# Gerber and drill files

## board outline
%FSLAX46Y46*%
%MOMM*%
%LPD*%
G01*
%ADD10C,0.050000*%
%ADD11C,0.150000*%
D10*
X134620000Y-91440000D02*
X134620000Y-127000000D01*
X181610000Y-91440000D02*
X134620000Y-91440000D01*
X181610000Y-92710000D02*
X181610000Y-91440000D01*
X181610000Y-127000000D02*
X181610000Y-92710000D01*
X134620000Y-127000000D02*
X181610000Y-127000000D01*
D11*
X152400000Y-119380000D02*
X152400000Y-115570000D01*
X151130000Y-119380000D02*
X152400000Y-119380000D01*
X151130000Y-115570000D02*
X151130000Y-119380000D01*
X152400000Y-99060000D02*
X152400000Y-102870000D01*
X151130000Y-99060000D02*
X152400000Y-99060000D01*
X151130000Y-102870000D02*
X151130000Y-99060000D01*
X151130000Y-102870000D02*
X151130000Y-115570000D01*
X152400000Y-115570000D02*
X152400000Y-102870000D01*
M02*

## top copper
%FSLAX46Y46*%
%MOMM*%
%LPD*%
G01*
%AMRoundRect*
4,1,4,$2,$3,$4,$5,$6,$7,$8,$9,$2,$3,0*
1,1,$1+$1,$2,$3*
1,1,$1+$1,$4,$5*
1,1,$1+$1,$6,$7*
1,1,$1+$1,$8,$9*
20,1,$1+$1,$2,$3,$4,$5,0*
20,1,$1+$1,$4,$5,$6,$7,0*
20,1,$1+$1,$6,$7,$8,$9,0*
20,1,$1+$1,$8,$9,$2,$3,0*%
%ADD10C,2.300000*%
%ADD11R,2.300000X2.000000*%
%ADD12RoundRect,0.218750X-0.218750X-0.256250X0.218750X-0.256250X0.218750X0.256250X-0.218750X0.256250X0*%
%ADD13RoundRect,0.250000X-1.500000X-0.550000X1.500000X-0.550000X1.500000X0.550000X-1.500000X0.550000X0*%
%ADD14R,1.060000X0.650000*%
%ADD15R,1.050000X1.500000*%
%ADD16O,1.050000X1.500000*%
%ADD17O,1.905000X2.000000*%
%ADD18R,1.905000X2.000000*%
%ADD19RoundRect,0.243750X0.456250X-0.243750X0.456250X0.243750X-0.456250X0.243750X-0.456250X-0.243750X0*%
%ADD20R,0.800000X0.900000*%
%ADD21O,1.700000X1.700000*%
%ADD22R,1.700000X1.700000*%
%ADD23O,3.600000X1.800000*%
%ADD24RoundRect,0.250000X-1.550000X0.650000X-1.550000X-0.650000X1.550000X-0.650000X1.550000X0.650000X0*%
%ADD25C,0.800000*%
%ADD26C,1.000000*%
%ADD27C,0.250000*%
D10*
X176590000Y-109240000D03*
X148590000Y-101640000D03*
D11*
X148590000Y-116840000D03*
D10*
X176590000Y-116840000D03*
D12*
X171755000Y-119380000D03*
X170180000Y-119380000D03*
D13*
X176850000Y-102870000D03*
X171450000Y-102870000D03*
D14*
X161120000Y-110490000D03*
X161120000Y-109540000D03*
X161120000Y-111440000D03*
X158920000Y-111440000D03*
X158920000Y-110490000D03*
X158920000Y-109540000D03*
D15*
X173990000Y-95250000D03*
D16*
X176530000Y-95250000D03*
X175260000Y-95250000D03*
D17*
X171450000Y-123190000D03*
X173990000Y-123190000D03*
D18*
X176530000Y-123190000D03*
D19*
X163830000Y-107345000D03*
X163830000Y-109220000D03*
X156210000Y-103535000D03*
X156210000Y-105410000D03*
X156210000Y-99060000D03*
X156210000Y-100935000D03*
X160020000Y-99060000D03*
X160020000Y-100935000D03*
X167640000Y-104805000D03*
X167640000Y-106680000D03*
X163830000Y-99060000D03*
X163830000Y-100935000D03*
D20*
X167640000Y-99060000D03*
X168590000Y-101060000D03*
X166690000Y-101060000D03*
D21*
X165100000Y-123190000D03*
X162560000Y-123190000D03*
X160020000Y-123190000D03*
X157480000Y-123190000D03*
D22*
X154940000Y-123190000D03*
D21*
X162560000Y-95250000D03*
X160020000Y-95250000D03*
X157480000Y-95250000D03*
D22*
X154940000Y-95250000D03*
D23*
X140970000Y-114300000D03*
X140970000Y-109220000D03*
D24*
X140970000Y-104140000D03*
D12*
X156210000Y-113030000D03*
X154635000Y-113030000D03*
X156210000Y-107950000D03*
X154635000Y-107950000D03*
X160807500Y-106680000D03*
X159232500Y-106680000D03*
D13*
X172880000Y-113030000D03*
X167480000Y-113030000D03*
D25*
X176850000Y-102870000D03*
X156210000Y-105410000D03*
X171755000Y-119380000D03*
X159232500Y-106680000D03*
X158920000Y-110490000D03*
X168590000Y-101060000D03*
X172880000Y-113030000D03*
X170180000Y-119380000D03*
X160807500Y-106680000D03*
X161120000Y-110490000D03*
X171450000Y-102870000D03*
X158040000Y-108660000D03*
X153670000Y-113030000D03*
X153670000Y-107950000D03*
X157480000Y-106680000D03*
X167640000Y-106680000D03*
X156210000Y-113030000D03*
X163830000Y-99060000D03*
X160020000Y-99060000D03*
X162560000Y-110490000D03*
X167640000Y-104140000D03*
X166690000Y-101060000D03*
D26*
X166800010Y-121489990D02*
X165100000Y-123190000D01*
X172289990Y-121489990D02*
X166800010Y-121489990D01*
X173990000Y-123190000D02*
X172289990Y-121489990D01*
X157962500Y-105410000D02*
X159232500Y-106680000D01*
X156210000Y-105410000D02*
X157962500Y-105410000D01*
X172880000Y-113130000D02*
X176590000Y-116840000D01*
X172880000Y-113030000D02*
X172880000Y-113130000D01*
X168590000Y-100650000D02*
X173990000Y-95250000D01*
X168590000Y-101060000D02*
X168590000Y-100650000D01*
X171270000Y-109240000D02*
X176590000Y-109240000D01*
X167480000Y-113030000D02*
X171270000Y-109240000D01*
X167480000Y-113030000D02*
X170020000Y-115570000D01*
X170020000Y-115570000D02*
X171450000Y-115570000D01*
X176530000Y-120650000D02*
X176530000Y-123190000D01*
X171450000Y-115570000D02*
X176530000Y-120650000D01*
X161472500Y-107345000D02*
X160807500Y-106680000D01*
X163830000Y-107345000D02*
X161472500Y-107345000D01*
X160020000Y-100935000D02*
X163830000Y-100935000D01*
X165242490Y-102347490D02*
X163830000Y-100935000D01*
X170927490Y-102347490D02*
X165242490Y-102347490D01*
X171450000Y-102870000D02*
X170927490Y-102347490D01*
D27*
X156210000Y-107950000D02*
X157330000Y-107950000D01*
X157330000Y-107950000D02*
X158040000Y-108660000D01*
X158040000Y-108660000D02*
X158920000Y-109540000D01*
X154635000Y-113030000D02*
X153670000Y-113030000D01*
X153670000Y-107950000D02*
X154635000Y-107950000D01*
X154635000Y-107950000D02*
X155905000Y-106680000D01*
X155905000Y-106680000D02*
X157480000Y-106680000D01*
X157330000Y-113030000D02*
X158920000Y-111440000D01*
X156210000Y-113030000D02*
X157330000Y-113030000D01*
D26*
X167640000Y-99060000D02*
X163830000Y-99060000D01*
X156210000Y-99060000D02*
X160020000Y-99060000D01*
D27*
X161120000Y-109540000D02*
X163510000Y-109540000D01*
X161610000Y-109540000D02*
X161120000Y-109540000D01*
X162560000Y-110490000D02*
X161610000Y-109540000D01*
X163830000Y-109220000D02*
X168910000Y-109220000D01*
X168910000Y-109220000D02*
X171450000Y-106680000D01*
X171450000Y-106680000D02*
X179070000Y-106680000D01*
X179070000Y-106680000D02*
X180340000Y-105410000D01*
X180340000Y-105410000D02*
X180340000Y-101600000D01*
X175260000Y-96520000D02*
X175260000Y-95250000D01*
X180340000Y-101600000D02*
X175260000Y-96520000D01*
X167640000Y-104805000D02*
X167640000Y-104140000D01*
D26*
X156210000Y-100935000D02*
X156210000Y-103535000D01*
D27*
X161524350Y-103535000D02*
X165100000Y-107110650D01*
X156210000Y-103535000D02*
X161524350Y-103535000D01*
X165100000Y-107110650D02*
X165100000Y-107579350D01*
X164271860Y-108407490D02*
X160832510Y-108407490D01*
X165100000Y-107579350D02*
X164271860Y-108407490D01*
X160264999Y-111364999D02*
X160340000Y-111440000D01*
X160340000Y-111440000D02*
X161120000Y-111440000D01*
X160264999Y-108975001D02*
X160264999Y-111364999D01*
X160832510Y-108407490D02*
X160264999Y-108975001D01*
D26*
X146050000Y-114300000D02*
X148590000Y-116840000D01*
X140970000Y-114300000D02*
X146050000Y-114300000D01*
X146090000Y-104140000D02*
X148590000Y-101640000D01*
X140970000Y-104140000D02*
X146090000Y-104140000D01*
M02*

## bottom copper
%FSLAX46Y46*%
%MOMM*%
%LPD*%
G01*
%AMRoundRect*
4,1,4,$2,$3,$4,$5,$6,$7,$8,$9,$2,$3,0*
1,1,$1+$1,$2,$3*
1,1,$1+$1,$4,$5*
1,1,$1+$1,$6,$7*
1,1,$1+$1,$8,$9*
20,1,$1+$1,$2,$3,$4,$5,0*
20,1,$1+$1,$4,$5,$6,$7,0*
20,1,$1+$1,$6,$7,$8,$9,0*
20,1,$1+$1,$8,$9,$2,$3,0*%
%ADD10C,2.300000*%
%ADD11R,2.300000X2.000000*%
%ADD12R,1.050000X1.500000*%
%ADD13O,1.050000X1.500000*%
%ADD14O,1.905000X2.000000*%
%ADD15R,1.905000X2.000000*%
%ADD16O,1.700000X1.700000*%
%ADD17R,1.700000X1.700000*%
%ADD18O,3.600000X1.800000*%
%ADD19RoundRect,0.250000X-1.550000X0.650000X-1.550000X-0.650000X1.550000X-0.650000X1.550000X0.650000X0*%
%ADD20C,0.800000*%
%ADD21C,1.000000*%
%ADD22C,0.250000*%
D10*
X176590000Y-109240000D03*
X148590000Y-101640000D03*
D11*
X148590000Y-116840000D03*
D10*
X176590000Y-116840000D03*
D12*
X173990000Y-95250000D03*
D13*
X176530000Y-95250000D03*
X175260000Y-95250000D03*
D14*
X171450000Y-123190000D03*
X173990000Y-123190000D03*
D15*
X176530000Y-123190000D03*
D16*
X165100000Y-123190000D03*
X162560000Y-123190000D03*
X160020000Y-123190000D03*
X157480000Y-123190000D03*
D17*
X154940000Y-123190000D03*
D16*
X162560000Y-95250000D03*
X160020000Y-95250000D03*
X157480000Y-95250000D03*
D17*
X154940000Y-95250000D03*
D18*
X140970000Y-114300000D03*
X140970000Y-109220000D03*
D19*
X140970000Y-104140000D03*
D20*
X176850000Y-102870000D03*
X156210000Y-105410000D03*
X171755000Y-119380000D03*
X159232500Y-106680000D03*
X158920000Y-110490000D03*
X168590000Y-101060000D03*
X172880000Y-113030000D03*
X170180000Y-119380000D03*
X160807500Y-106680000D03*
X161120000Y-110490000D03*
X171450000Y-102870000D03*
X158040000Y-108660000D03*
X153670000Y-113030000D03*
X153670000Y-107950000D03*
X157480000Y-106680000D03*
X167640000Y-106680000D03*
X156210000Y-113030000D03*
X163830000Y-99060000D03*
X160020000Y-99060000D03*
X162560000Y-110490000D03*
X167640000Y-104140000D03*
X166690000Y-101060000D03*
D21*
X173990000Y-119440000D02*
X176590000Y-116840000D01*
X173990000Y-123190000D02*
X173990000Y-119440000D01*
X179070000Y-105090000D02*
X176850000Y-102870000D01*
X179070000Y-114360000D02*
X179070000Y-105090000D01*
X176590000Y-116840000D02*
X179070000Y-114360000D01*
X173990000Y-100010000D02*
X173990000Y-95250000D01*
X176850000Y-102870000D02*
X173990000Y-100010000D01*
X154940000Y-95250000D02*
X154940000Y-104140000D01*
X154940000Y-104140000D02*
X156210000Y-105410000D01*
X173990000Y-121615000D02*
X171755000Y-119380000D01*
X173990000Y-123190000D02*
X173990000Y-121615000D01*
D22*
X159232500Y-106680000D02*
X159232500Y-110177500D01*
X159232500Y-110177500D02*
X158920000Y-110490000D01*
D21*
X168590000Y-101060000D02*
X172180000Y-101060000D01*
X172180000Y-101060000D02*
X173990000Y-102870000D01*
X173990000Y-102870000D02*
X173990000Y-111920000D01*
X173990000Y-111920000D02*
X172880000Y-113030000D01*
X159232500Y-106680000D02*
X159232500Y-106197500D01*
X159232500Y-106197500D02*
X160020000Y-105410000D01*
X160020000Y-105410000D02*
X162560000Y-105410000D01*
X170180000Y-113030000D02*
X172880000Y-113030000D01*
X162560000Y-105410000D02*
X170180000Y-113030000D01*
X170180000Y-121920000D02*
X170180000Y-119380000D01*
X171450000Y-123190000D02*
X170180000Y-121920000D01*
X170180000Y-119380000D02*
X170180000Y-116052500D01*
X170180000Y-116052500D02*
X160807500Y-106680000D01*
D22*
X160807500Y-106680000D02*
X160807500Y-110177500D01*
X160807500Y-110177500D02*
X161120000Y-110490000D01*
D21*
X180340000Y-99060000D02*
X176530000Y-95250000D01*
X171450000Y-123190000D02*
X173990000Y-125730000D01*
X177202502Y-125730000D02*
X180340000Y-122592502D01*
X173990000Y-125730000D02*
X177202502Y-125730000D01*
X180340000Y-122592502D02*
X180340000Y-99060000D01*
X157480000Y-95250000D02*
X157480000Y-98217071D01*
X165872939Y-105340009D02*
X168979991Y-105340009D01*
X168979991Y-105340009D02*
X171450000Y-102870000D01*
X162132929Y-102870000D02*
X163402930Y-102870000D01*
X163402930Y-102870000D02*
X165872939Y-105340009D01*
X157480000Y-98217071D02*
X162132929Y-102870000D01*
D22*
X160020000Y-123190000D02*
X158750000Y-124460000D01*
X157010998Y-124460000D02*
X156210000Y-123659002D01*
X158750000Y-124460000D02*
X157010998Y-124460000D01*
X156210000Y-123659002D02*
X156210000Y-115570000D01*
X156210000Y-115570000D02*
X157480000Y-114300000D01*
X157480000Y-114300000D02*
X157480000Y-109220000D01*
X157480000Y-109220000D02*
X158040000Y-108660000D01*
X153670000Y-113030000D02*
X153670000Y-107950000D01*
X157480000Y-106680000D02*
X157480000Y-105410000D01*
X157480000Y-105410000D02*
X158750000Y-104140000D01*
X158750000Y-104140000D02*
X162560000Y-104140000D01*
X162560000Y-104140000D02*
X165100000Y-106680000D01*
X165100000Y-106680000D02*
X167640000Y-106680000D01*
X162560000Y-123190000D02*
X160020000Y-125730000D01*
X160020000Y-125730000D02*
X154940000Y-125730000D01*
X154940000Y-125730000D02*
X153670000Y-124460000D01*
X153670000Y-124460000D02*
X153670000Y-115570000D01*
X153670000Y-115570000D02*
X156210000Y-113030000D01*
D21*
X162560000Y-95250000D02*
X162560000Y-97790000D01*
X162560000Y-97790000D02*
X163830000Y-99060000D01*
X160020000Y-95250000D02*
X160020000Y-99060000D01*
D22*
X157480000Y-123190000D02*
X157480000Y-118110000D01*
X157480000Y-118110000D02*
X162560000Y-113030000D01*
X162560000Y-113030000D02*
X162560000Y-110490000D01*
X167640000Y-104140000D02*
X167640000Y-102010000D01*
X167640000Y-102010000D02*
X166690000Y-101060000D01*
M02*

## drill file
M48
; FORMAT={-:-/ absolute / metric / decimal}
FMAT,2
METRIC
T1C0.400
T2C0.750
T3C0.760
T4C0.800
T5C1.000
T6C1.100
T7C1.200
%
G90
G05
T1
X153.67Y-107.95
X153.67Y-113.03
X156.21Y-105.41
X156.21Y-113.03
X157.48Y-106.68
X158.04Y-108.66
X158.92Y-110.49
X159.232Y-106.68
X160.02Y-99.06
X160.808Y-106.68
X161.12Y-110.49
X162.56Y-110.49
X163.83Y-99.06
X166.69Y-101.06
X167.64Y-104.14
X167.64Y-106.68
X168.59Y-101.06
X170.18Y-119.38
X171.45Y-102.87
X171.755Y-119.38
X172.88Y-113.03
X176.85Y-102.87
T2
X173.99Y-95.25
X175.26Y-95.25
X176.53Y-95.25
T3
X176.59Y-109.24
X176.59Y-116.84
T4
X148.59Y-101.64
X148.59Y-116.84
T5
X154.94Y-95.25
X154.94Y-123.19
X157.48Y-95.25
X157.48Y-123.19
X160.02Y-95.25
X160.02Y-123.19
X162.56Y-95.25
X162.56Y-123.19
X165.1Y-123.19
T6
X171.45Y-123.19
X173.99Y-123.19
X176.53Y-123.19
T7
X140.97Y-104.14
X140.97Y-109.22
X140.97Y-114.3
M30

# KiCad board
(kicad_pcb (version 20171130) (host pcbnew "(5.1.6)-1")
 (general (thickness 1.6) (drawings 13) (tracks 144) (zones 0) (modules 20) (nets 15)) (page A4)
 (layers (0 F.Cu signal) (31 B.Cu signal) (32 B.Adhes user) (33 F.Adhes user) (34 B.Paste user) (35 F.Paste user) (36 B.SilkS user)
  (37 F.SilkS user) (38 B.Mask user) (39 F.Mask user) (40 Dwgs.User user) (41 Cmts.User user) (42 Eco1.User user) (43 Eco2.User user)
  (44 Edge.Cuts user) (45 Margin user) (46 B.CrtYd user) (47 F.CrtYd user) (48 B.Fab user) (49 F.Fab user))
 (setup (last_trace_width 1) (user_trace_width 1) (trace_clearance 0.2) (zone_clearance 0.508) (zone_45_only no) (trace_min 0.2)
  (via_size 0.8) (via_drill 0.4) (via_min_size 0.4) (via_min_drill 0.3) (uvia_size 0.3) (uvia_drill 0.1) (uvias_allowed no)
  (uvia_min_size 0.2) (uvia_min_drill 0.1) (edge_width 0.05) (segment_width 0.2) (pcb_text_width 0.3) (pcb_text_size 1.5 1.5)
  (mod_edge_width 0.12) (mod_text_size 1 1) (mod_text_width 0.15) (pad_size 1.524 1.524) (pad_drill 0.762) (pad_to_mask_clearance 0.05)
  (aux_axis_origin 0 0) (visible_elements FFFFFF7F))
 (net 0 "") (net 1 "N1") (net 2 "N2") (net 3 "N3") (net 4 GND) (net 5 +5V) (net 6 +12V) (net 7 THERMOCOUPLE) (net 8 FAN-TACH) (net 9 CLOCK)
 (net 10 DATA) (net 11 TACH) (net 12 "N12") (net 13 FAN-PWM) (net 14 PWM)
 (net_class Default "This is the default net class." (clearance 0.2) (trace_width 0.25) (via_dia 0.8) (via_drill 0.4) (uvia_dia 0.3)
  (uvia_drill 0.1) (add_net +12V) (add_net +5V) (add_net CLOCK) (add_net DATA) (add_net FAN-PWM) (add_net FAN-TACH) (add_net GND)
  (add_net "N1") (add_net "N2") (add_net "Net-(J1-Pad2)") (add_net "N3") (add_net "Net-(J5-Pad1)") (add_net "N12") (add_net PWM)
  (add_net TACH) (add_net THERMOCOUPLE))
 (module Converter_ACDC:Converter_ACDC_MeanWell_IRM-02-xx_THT (layer B.Cu) (at 148.59 116.84)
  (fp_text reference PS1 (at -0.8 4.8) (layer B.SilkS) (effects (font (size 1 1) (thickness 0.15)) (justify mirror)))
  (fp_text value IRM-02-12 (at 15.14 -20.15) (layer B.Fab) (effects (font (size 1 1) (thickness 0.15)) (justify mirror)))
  (pad 4 thru_hole circle (at 28 -7.6) (size 2.3 2.3) (drill 0.76) (layers *.Cu *.Mask) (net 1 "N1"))
  (pad 2 thru_hole circle (at 0 -15.2) (size 2.3 2.3) (drill 0.8) (layers *.Cu *.Mask) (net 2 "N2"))
  (pad 1 thru_hole rect (at 0 0) (size 2.3 2) (drill 0.8) (layers *.Cu *.Mask) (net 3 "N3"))
  (pad 3 thru_hole circle (at 28 0) (size 2.3 2.3) (drill 0.76) (layers *.Cu *.Mask) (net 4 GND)))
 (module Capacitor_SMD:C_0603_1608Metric (layer F.Cu) (at 170.9675 119.38)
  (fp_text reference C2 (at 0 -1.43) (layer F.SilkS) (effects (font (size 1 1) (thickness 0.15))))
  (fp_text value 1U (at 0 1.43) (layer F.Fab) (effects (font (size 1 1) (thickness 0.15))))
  (pad 2 smd roundrect (at 0.7875 0) (size 0.875 0.95) (layers F.Cu F.Paste F.Mask) (roundrect_rratio 0.25) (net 4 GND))
  (pad 1 smd roundrect (at -0.7875 0) (size 0.875 0.95) (layers F.Cu F.Paste F.Mask) (roundrect_rratio 0.25) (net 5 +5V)))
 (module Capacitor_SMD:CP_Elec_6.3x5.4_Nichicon (layer F.Cu) (at 174.15 102.87)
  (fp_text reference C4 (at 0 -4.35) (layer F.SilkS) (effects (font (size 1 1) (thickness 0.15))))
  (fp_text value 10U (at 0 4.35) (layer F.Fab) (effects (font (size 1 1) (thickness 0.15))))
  (pad 2 smd roundrect (at 2.7 0) (size 3.5 1.6) (layers F.Cu F.Paste F.Mask) (roundrect_rratio 0.15625) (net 4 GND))
  (pad 1 smd roundrect (at -2.7 0) (size 3.5 1.6) (layers F.Cu F.Paste F.Mask) (roundrect_rratio 0.15625) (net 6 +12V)))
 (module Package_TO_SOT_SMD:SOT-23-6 (layer F.Cu) (at 160.02 110.49)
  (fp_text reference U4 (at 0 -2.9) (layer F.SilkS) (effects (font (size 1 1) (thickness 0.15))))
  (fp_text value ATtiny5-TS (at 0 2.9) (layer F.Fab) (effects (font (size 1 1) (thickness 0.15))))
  (pad 5 smd rect (at 1.1 0) (size 1.06 0.65) (layers F.Cu F.Paste F.Mask) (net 5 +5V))
  (pad 6 smd rect (at 1.1 -0.95) (size 1.06 0.65) (layers F.Cu F.Paste F.Mask) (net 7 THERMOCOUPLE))
  (pad 4 smd rect (at 1.1 0.95) (size 1.06 0.65) (layers F.Cu F.Paste F.Mask) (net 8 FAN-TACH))
  (pad 3 smd rect (at -1.1 0.95) (size 1.06 0.65) (layers F.Cu F.Paste F.Mask) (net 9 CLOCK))
  (pad 2 smd rect (at -1.1 0) (size 1.06 0.65) (layers F.Cu F.Paste F.Mask) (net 4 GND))
  (pad 1 smd rect (at -1.1 -0.95) (size 1.06 0.65) (layers F.Cu F.Paste F.Mask) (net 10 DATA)))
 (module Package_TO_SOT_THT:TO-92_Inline (layer F.Cu) (at 173.99 95.25)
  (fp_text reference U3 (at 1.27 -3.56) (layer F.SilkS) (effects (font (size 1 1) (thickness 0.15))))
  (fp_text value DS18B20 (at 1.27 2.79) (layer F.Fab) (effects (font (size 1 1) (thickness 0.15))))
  (pad 1 thru_hole rect (at 0 0) (size 1.05 1.5) (drill 0.75) (layers *.Cu *.Mask) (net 4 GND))
  (pad 3 thru_hole oval (at 2.54 0) (size 1.05 1.5) (drill 0.75) (layers *.Cu *.Mask) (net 5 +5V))
  (pad 2 thru_hole oval (at 1.27 0) (size 1.05 1.5) (drill 0.75) (layers *.Cu *.Mask) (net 7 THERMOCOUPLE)))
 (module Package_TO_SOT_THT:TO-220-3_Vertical (layer F.Cu) (at 176.53 123.19 180)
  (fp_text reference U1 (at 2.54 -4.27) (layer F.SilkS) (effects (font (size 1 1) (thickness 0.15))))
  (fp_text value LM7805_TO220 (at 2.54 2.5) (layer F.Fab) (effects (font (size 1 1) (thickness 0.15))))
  (pad 3 thru_hole oval (at 5.08 0 180) (size 1.905 2) (drill 1.1) (layers *.Cu *.Mask) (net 5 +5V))
  (pad 2 thru_hole oval (at 2.54 0 180) (size 1.905 2) (drill 1.1) (layers *.Cu *.Mask) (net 4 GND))
  (pad 1 thru_hole rect (at 0 0 180) (size 1.905 2) (drill 1.1) (layers *.Cu *.Mask) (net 1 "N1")))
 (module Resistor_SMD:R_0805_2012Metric (layer F.Cu) (at 163.83 108.2825 90)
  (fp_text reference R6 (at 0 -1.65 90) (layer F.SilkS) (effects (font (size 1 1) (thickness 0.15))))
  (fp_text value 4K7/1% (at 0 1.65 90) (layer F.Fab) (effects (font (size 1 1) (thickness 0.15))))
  (pad 2 smd roundrect (at 0.9375 0 90) (size 0.975 1.4) (layers F.Cu F.Paste F.Mask) (roundrect_rratio 0.25) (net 5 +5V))
  (pad 1 smd roundrect (at -0.9375 0 90) (size 0.975 1.4) (layers F.Cu F.Paste F.Mask) (roundrect_rratio 0.25) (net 7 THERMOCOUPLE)))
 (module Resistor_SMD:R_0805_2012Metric (layer F.Cu) (at 156.21 104.4725 90)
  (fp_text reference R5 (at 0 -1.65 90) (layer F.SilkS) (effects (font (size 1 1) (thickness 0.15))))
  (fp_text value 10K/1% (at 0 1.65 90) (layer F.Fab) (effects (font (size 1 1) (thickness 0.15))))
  (pad 2 smd roundrect (at 0.9375 0 90) (size 0.975 1.4) (layers F.Cu F.Paste F.Mask) (roundrect_rratio 0.25) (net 8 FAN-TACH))
  (pad 1 smd roundrect (at -0.9375 0 90) (size 0.975 1.4) (layers F.Cu F.Paste F.Mask) (roundrect_rratio 0.25) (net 4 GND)))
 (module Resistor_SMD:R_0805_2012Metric (layer F.Cu) (at 156.21 99.9975 90)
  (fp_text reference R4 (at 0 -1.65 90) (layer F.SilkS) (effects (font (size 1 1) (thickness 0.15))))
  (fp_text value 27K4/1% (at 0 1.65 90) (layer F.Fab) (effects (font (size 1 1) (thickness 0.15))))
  (pad 2 smd roundrect (at 0.9375 0 90) (size 0.975 1.4) (layers F.Cu F.Paste F.Mask) (roundrect_rratio 0.25) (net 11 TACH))
  (pad 1 smd roundrect (at -0.9375 0 90) (size 0.975 1.4) (layers F.Cu F.Paste F.Mask) (roundrect_rratio 0.25) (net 8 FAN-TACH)))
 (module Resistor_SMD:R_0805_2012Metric (layer F.Cu) (at 160.02 99.9975 90)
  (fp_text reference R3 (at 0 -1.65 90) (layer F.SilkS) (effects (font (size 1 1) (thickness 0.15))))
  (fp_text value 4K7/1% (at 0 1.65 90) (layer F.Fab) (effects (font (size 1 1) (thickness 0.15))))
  (pad 2 smd roundrect (at 0.9375 0 90) (size 0.975 1.4) (layers F.Cu F.Paste F.Mask) (roundrect_rratio 0.25) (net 11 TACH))
  (pad 1 smd roundrect (at -0.9375 0 90) (size 0.975 1.4) (layers F.Cu F.Paste F.Mask) (roundrect_rratio 0.25) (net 6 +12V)))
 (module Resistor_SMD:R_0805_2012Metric (layer F.Cu) (at 167.64 105.7425 90)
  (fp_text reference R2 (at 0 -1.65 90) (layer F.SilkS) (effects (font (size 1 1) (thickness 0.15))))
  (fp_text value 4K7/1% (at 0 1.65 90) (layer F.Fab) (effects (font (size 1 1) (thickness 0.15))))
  (pad 2 smd roundrect (at 0.9375 0 90) (size 0.975 1.4) (layers F.Cu F.Paste F.Mask) (roundrect_rratio 0.25) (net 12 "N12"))
  (pad 1 smd roundrect (at -0.9375 0 90) (size 0.975 1.4) (layers F.Cu F.Paste F.Mask) (roundrect_rratio 0.25) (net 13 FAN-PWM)))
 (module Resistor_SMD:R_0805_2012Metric (layer F.Cu) (at 163.83 99.9975 90)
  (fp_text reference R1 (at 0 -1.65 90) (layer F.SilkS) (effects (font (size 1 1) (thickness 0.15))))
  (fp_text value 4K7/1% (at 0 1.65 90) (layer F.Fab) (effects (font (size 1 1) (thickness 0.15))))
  (pad 2 smd roundrect (at 0.9375 0 90) (size 0.975 1.4) (layers F.Cu F.Paste F.Mask) (roundrect_rratio 0.25) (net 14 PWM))
  (pad 1 smd roundrect (at -0.9375 0 90) (size 0.975 1.4) (layers F.Cu F.Paste F.Mask) (roundrect_rratio 0.25) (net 6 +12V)))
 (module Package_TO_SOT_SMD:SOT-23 (layer F.Cu) (at 167.64 100.06 90)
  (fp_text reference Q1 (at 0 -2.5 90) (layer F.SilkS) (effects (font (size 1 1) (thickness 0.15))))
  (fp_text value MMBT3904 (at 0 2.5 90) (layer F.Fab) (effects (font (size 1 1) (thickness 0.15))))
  (pad 3 smd rect (at 1 0 90) (size 0.9 0.8) (layers F.Cu F.Paste F.Mask) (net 14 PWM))
  (pad 2 smd rect (at -1 0.95 90) (size 0.9 0.8) (layers F.Cu F.Paste F.Mask) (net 4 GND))
  (pad 1 smd rect (at -1 -0.95 90) (size 0.9 0.8) (layers F.Cu F.Paste F.Mask) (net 12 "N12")))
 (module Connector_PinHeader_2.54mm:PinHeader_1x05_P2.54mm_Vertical (layer F.Cu) (at 154.94 123.19 90)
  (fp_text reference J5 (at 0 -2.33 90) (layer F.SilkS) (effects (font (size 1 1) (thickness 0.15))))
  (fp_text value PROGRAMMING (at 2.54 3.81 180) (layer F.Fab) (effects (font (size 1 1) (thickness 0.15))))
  (pad 5 thru_hole oval (at 0 10.16 90) (size 1.7 1.7) (drill 1) (layers *.Cu *.Mask) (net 4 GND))
  (pad 4 thru_hole oval (at 0 7.62 90) (size 1.7 1.7) (drill 1) (layers *.Cu *.Mask) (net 9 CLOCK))
  (pad 3 thru_hole oval (at 0 5.08 90) (size 1.7 1.7) (drill 1) (layers *.Cu *.Mask) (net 10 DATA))
  (pad 2 thru_hole oval (at 0 2.54 90) (size 1.7 1.7) (drill 1) (layers *.Cu *.Mask) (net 7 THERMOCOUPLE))
  (pad 1 thru_hole rect (at 0 0 90) (size 1.7 1.7) (drill 1) (layers *.Cu *.Mask)))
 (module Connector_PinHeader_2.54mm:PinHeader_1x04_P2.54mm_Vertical (layer F.Cu) (at 154.94 95.25 90)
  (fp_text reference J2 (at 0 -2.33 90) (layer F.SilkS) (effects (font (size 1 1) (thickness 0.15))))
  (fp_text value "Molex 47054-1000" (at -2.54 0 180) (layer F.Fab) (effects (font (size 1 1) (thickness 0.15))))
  (pad 4 thru_hole oval (at 0 7.62 90) (size 1.7 1.7) (drill 1) (layers *.Cu *.Mask) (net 14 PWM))
  (pad 3 thru_hole oval (at 0 5.08 90) (size 1.7 1.7) (drill 1) (layers *.Cu *.Mask) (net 11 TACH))
  (pad 2 thru_hole oval (at 0 2.54 90) (size 1.7 1.7) (drill 1) (layers *.Cu *.Mask) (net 6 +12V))
  (pad 1 thru_hole rect (at 0 0 90) (size 1.7 1.7) (drill 1) (layers *.Cu *.Mask) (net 4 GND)))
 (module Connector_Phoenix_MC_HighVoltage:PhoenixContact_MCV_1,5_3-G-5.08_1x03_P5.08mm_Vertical (layer B.Cu) (at 140.97 104.14 270)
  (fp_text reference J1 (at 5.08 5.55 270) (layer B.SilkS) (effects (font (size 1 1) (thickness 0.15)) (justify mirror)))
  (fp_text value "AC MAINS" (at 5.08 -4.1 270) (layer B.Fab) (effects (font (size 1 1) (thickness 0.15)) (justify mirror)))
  (pad 3 thru_hole oval (at 10.16 0 270) (size 1.8 3.6) (drill 1.2) (layers *.Cu *.Mask) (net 3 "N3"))
  (pad 2 thru_hole oval (at 5.08 0 270) (size 1.8 3.6) (drill 1.2) (layers *.Cu *.Mask))
  (pad 1 thru_hole roundrect (at 0 0 270) (size 1.8 3.6) (drill 1.2) (layers *.Cu *.Mask) (roundrect_rratio 0.138889) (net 2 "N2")))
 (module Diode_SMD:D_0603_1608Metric (layer F.Cu) (at 155.4225 113.03)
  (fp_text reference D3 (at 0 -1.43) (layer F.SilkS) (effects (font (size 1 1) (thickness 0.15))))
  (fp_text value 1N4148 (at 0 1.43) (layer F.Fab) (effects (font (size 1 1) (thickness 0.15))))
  (pad 2 smd roundrect (at 0.7875 0) (size 0.875 0.95) (layers F.Cu F.Paste F.Mask) (roundrect_rratio 0.25) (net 9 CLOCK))
  (pad 1 smd roundrect (at -0.7875 0) (size 0.875 0.95) (layers F.Cu F.Paste F.Mask) (roundrect_rratio 0.25) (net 13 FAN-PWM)))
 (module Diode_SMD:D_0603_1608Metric (layer F.Cu) (at 155.4225 107.95)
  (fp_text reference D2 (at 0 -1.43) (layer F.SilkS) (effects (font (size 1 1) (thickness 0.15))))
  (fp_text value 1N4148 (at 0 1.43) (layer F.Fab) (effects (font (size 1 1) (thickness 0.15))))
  (pad 2 smd roundrect (at 0.7875 0) (size 0.875 0.95) (layers F.Cu F.Paste F.Mask) (roundrect_rratio 0.25) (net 10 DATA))
  (pad 1 smd roundrect (at -0.7875 0) (size 0.875 0.95) (layers F.Cu F.Paste F.Mask) (roundrect_rratio 0.25) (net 13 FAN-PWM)))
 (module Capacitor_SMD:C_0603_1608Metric (layer F.Cu) (at 160.02 106.68)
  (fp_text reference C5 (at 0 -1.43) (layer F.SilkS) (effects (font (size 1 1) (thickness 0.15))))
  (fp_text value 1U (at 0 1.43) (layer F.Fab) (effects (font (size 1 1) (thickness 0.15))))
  (pad 2 smd roundrect (at 0.7875 0) (size 0.875 0.95) (layers F.Cu F.Paste F.Mask) (roundrect_rratio 0.25) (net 5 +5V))
  (pad 1 smd roundrect (at -0.7875 0) (size 0.875 0.95) (layers F.Cu F.Paste F.Mask) (roundrect_rratio 0.25) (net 4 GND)))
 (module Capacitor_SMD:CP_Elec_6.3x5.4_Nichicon (layer F.Cu) (at 170.18 113.03)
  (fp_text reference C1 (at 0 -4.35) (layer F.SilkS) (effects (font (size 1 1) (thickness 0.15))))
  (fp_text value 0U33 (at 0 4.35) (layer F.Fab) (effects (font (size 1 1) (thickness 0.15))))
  (pad 2 smd roundrect (at 2.7 0) (size 3.5 1.6) (layers F.Cu F.Paste F.Mask) (roundrect_rratio 0.15625) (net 4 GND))
  (pad 1 smd roundrect (at -2.7 0) (size 3.5 1.6) (layers F.Cu F.Paste F.Mask) (roundrect_rratio 0.15625) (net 1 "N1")))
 (gr_line (start 134.62 91.44) (end 134.62 127) (layer Edge.Cuts) (width 0.05))
 (gr_line (start 181.61 91.44) (end 134.62 91.44) (layer Edge.Cuts) (width 0.05))
 (gr_line (start 181.61 92.71) (end 181.61 91.44) (layer Edge.Cuts) (width 0.05))
 (gr_line (start 181.61 127) (end 181.61 92.71) (layer Edge.Cuts) (width 0.05))
 (gr_line (start 134.62 127) (end 181.61 127) (layer Edge.Cuts) (width 0.05))
 (gr_line (start 152.4 119.38) (end 152.4 115.57) (layer Edge.Cuts) (width 0.15))
 (gr_line (start 151.13 119.38) (end 152.4 119.38) (layer Edge.Cuts) (width 0.15))
 (gr_line (start 151.13 115.57) (end 151.13 119.38) (layer Edge.Cuts) (width 0.15))
 (gr_line (start 152.4 99.06) (end 152.4 102.87) (layer Edge.Cuts) (width 0.15))
 (gr_line (start 151.13 99.06) (end 152.4 99.06) (layer Edge.Cuts) (width 0.15))
 (gr_line (start 151.13 102.87) (end 151.13 99.06) (layer Edge.Cuts) (width 0.15))
 (gr_line (start 151.13 102.87) (end 151.13 115.57) (layer Edge.Cuts) (width 0.15))
 (gr_line (start 152.4 115.57) (end 152.4 102.87) (layer Edge.Cuts) (width 0.15))
 (segment (start 173.99 119.44) (end 176.59 116.84) (width 1) (layer B.Cu) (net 4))
 (segment (start 173.99 123.19) (end 173.99 119.44) (width 1) (layer B.Cu) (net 4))
 (segment (start 166.80001 121.48999) (end 165.1 123.19) (width 1) (layer F.Cu) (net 4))
 (segment (start 172.28999 121.48999) (end 166.80001 121.48999) (width 1) (layer F.Cu) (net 4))
 (segment (start 173.99 123.19) (end 172.28999 121.48999) (width 1) (layer F.Cu) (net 4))
 (segment (start 179.07 105.09) (end 176.85 102.87) (width 1) (layer B.Cu) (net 4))
 (segment (start 179.07 114.36) (end 179.07 105.09) (width 1) (layer B.Cu) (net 4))
 (segment (start 176.59 116.84) (end 179.07 114.36) (width 1) (layer B.Cu) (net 4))
 (via (at 176.85 102.87) (size 0.8) (drill 0.4) (layers F.Cu B.Cu) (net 4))
 (segment (start 173.99 100.01) (end 173.99 95.25) (width 1) (layer B.Cu) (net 4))
 (segment (start 176.85 102.87) (end 173.99 100.01) (width 1) (layer B.Cu) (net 4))
 (via (at 156.21 105.41) (size 0.8) (drill 0.4) (layers F.Cu B.Cu) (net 4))
 (segment (start 154.94 95.25) (end 154.94 104.14) (width 1) (layer B.Cu) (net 4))
 (segment (start 154.94 104.14) (end 156.21 105.41) (width 1) (layer B.Cu) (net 4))
 (segment (start 157.9625 105.41) (end 159.2325 106.68) (width 1) (layer F.Cu) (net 4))
 (segment (start 156.21 105.41) (end 157.9625 105.41) (width 1) (layer F.Cu) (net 4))
 (segment (start 173.99 121.615) (end 171.755 119.38) (width 1) (layer B.Cu) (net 4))
 (via (at 171.755 119.38) (size 0.8) (drill 0.4) (layers F.Cu B.Cu) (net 4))
 (segment (start 173.99 123.19) (end 173.99 121.615) (width 1) (layer B.Cu) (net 4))
 (segment (start 172.88 113.13) (end 176.59 116.84) (width 1) (layer F.Cu) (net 4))
 (segment (start 172.88 113.03) (end 172.88 113.13) (width 1) (layer F.Cu) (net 4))
 (segment (start 168.59 100.65) (end 173.99 95.25) (width 1) (layer F.Cu) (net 4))
 (segment (start 168.59 101.06) (end 168.59 100.65) (width 1) (layer F.Cu) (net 4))
 (via (at 159.2325 106.68) (size 0.8) (drill 0.4) (layers F.Cu B.Cu) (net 4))
 (segment (start 159.2325 106.68) (end 159.2325 110.1775) (width 0.25) (layer B.Cu) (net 4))
 (via (at 158.92 110.49) (size 0.8) (drill 0.4) (layers F.Cu B.Cu) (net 4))
 (segment (start 159.2325 110.1775) (end 158.92 110.49) (width 0.25) (layer B.Cu) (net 4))
 (via (at 168.59 101.06) (size 0.8) (drill 0.4) (layers F.Cu B.Cu) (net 4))
 (segment (start 168.59 101.06) (end 172.18 101.06) (width 1) (layer B.Cu) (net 4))
 (segment (start 172.18 101.06) (end 173.99 102.87) (width 1) (layer B.Cu) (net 4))
 (via (at 172.88 113.03) (size 0.8) (drill 0.4) (layers F.Cu B.Cu) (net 4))
 (segment (start 173.99 102.87) (end 173.99 111.92) (width 1) (layer B.Cu) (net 4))
 (segment (start 173.99 111.92) (end 172.88 113.03) (width 1) (layer B.Cu) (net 4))
 (segment (start 159.2325 106.68) (end 159.2325 106.1975) (width 1) (layer B.Cu) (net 4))
 (segment (start 159.2325 106.1975) (end 160.02 105.41) (width 1) (layer B.Cu) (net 4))
 (segment (start 160.02 105.41) (end 162.56 105.41) (width 1) (layer B.Cu) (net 4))
 (segment (start 170.18 113.03) (end 172.88 113.03) (width 1) (layer B.Cu) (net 4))
 (segment (start 162.56 105.41) (end 170.18 113.03) (width 1) (layer B.Cu) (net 4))
 (segment (start 171.27 109.24) (end 176.59 109.24) (width 1) (layer F.Cu) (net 1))
 (segment (start 167.48 113.03) (end 171.27 109.24) (width 1) (layer F.Cu) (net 1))
 (segment (start 167.48 113.03) (end 170.02 115.57) (width 1) (layer F.Cu) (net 1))
 (segment (start 170.02 115.57) (end 171.45 115.57) (width 1) (layer F.Cu) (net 1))
 (segment (start 176.53 120.65) (end 176.53 123.19) (width 1) (layer F.Cu) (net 1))
 (segment (start 171.45 115.57) (end 176.53 120.65) (width 1) (layer F.Cu) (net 1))
 (segment (start 161.4725 107.345) (end 160.8075 106.68) (width 1) (layer F.Cu) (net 5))
 (segment (start 163.83 107.345) (end 161.4725 107.345) (width 1) (layer F.Cu) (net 5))
 (via (at 170.18 119.38) (size 0.8) (drill 0.4) (layers F.Cu B.Cu) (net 5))
 (segment (start 170.18 121.92) (end 170.18 119.38) (width 1) (layer B.Cu) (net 5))
 (segment (start 171.45 123.19) (end 170.18 121.92) (width 1) (layer B.Cu) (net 5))
 (via (at 160.8075 106.68) (size 0.8) (drill 0.4) (layers F.Cu B.Cu) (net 5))
 (segment (start 170.18 119.38) (end 170.18 116.0525) (width 1) (layer B.Cu) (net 5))
 (segment (start 170.18 116.0525) (end 160.8075 106.68) (width 1) (layer B.Cu) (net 5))
 (via (at 161.12 110.49) (size 0.8) (drill 0.4) (layers F.Cu B.Cu) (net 5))
 (segment (start 160.8075 106.68) (end 160.8075 110.1775) (width 0.25) (layer B.Cu) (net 5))
 (segment (start 160.8075 110.1775) (end 161.12 110.49) (width 0.25) (layer B.Cu) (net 5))
 (segment (start 180.34 99.06) (end 176.53 95.25) (width 1) (layer B.Cu) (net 5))
 (segment (start 171.45 123.19) (end 173.99 125.73) (width 1) (layer B.Cu) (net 5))
 (segment (start 177.202502 125.73) (end 180.34 122.592502) (width 1) (layer B.Cu) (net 5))
 (segment (start 173.99 125.73) (end 177.202502 125.73) (width 1) (layer B.Cu) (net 5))
 (segment (start 180.34 122.592502) (end 180.34 99.06) (width 1) (layer B.Cu) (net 5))
 (segment (start 160.02 100.935) (end 163.83 100.935) (width 1) (layer F.Cu) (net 6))
 (segment (start 165.24249 102.34749) (end 163.83 100.935) (width 1) (layer F.Cu) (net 6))
 (segment (start 170.92749 102.34749) (end 165.24249 102.34749) (width 1) (layer F.Cu) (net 6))
 (segment (start 171.45 102.87) (end 170.92749 102.34749) (width 1) (layer F.Cu) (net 6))
 (via (at 171.45 102.87) (size 0.8) (drill 0.4) (layers F.Cu B.Cu) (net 6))
 (segment (start 157.48 95.25) (end 157.48 98.217071) (width 1) (layer B.Cu) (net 6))
 (segment (start 165.872939 105.340009) (end 168.979991 105.340009) (width 1) (layer B.Cu) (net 6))
 (segment (start 168.979991 105.340009) (end 171.45 102.87) (width 1) (layer B.Cu) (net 6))
 (segment (start 162.132929 102.87) (end 163.40293 102.87) (width 1) (layer B.Cu) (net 6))
 (segment (start 163.40293 102.87) (end 165.872939 105.340009) (width 1) (layer B.Cu) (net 6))
 (segment (start 157.48 98.217071) (end 162.132929 102.87) (width 1) (layer B.Cu) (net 6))
 (segment (start 156.21 107.95) (end 157.33 107.95) (width 0.25) (layer F.Cu) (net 10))
 (segment (start 160.02 123.19) (end 158.75 124.46) (width 0.25) (layer B.Cu) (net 10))
 (segment (start 157.010998 124.46) (end 156.21 123.659002) (width 0.25) (layer B.Cu) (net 10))
 (segment (start 158.75 124.46) (end 157.010998 124.46) (width 0.25) (layer B.Cu) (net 10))
 (segment (start 156.21 123.659002) (end 156.21 115.57) (width 0.25) (layer B.Cu) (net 10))
 (segment (start 156.21 115.57) (end 157.48 114.3) (width 0.25) (layer B.Cu) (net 10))
 (segment (start 157.48 114.3) (end 157.48 109.22) (width 0.25) (layer B.Cu) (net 10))
 (via (at 158.04 108.66) (size 0.8) (drill 0.4) (layers F.Cu B.Cu) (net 10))
 (segment (start 157.48 109.22) (end 158.04 108.66) (width 0.25) (layer B.Cu) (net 10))
 (segment (start 157.33 107.95) (end 158.04 108.66) (width 0.25) (layer F.Cu) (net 10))
 (segment (start 158.04 108.66) (end 158.92 109.54) (width 0.25) (layer F.Cu) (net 10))
 (via (at 153.67 113.03) (size 0.8) (drill 0.4) (layers F.Cu B.Cu) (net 13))
 (segment (start 154.635 113.03) (end 153.67 113.03) (width 0.25) (layer F.Cu) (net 13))
 (via (at 153.67 107.95) (size 0.8) (drill 0.4) (layers F.Cu B.Cu) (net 13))
 (segment (start 153.67 113.03) (end 153.67 107.95) (width 0.25) (layer B.Cu) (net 13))
 (segment (start 153.67 107.95) (end 154.635 107.95) (width 0.25) (layer F.Cu) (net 13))
 (segment (start 154.635 107.95) (end 155.905 106.68) (width 0.25) (layer F.Cu) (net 13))
 (via (at 157.48 106.68) (size 0.8) (drill 0.4) (layers F.Cu B.Cu) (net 13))
 (segment (start 155.905 106.68) (end 157.48 106.68) (width 0.25) (layer F.Cu) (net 13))
 (segment (start 157.48 106.68) (end 157.48 105.41) (width 0.25) (layer B.Cu) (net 13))
 (segment (start 157.48 105.41) (end 158.75 104.14) (width 0.25) (layer B.Cu) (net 13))
 (segment (start 158.75 104.14) (end 162.56 104.14) (width 0.25) (layer B.Cu) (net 13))
 (segment (start 162.56 104.14) (end 165.1 106.68) (width 0.25) (layer B.Cu) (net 13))
 (segment (start 165.1 106.68) (end 167.64 106.68) (width 0.25) (layer B.Cu) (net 13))
 (via (at 167.64 106.68) (size 0.8) (drill 0.4) (layers F.Cu B.Cu) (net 13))
 (segment (start 157.33 113.03) (end 158.92 111.44) (width 0.25) (layer F.Cu) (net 9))
 (segment (start 156.21 113.03) (end 157.33 113.03) (width 0.25) (layer F.Cu) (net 9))
 (segment (start 162.56 123.19) (end 160.02 125.73) (width 0.25) (layer B.Cu) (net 9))
 (segment (start 160.02 125.73) (end 154.94 125.73) (width 0.25) (layer B.Cu) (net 9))
 (segment (start 154.94 125.73) (end 153.67 124.46) (width 0.25) (layer B.Cu) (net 9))
 (segment (start 153.67 124.46) (end 153.67 115.57) (width 0.25) (layer B.Cu) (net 9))
 (via (at 156.21 113.03) (size 0.8) (drill 0.4) (layers F.Cu B.Cu) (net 9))
 (segment (start 153.67 115.57) (end 156.21 113.03) (width 0.25) (layer B.Cu) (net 9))
 (via (at 163.83 99.06) (size 0.8) (drill 0.4) (layers F.Cu B.Cu) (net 14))
 (segment (start 162.56 95.25) (end 162.56 97.79) (width 1) (layer B.Cu) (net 14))
 (segment (start 162.56 97.79) (end 163.83 99.06) (width 1) (layer B.Cu) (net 14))
 (segment (start 167.64 99.06) (end 163.83 99.06) (width 1) (layer F.Cu) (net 14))
 (segment (start 156.21 99.06) (end 160.02 99.06) (width 1) (layer F.Cu) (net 11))
 (via (at 160.02 99.06) (size 0.8) (drill 0.4) (layers F.Cu B.Cu) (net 11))
 (segment (start 160.02 95.25) (end 160.02 99.06) (width 1) (layer B.Cu) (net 11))
 (segment (start 161.12 109.54) (end 163.51 109.54) (width 0.25) (layer F.Cu) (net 7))
 (segment (start 157.48 123.19) (end 157.48 118.11) (width 0.25) (layer B.Cu) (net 7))
 (segment (start 157.48 118.11) (end 162.56 113.03) (width 0.25) (layer B.Cu) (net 7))
 (via (at 162.56 110.49) (size 0.8) (drill 0.4) (layers F.Cu B.Cu) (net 7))
 (segment (start 162.56 113.03) (end 162.56 110.49) (width 0.25) (layer B.Cu) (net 7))
 (segment (start 161.61 109.54) (end 161.12 109.54) (width 0.25) (layer F.Cu) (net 7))
 (segment (start 162.56 110.49) (end 161.61 109.54) (width 0.25) (layer F.Cu) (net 7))
 (segment (start 163.83 109.22) (end 168.91 109.22) (width 0.25) (layer F.Cu) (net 7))
 (segment (start 168.91 109.22) (end 171.45 106.68) (width 0.25) (layer F.Cu) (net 7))
 (segment (start 171.45 106.68) (end 179.07 106.68) (width 0.25) (layer F.Cu) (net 7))
 (segment (start 179.07 106.68) (end 180.34 105.41) (width 0.25) (layer F.Cu) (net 7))
 (segment (start 180.34 105.41) (end 180.34 101.6) (width 0.25) (layer F.Cu) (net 7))
 (segment (start 175.26 96.52) (end 175.26 95.25) (width 0.25) (layer F.Cu) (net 7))
 (segment (start 180.34 101.6) (end 175.26 96.52) (width 0.25) (layer F.Cu) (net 7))
 (via (at 167.64 104.14) (size 0.8) (drill 0.4) (layers F.Cu B.Cu) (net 12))
 (segment (start 167.64 104.805) (end 167.64 104.14) (width 0.25) (layer F.Cu) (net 12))
 (via (at 166.69 101.06) (size 0.8) (drill 0.4) (layers F.Cu B.Cu) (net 12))
 (segment (start 167.64 104.14) (end 167.64 102.01) (width 0.25) (layer B.Cu) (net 12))
 (segment (start 167.64 102.01) (end 166.69 101.06) (width 0.25) (layer B.Cu) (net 12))
 (segment (start 156.21 100.935) (end 156.21 103.535) (width 1) (layer F.Cu) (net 8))
 (segment (start 161.52435 103.535) (end 165.1 107.11065) (width 0.25) (layer F.Cu) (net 8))
 (segment (start 156.21 103.535) (end 161.52435 103.535) (width 0.25) (layer F.Cu) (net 8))
 (segment (start 165.1 107.11065) (end 165.1 107.57935) (width 0.25) (layer F.Cu) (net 8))
 (segment (start 164.27186 108.40749) (end 160.83251 108.40749) (width 0.25) (layer F.Cu) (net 8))
 (segment (start 165.1 107.57935) (end 164.27186 108.40749) (width 0.25) (layer F.Cu) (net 8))
 (segment (start 160.264999 111.364999) (end 160.34 111.44) (width 0.25) (layer F.Cu) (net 8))
 (segment (start 160.34 111.44) (end 161.12 111.44) (width 0.25) (layer F.Cu) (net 8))
 (segment (start 160.264999 108.975001) (end 160.264999 111.364999) (width 0.25) (layer F.Cu) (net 8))
 (segment (start 160.83251 108.40749) (end 160.264999 108.975001) (width 0.25) (layer F.Cu) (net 8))
 (segment (start 146.05 114.3) (end 148.59 116.84) (width 1) (layer F.Cu) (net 3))
 (segment (start 140.97 114.3) (end 146.05 114.3) (width 1) (layer F.Cu) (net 3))
 (segment (start 146.09 104.14) (end 148.59 101.64) (width 1) (layer F.Cu) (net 2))
 (segment (start 140.97 104.14) (end 146.09 104.14) (width 1) (layer F.Cu) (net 2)))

